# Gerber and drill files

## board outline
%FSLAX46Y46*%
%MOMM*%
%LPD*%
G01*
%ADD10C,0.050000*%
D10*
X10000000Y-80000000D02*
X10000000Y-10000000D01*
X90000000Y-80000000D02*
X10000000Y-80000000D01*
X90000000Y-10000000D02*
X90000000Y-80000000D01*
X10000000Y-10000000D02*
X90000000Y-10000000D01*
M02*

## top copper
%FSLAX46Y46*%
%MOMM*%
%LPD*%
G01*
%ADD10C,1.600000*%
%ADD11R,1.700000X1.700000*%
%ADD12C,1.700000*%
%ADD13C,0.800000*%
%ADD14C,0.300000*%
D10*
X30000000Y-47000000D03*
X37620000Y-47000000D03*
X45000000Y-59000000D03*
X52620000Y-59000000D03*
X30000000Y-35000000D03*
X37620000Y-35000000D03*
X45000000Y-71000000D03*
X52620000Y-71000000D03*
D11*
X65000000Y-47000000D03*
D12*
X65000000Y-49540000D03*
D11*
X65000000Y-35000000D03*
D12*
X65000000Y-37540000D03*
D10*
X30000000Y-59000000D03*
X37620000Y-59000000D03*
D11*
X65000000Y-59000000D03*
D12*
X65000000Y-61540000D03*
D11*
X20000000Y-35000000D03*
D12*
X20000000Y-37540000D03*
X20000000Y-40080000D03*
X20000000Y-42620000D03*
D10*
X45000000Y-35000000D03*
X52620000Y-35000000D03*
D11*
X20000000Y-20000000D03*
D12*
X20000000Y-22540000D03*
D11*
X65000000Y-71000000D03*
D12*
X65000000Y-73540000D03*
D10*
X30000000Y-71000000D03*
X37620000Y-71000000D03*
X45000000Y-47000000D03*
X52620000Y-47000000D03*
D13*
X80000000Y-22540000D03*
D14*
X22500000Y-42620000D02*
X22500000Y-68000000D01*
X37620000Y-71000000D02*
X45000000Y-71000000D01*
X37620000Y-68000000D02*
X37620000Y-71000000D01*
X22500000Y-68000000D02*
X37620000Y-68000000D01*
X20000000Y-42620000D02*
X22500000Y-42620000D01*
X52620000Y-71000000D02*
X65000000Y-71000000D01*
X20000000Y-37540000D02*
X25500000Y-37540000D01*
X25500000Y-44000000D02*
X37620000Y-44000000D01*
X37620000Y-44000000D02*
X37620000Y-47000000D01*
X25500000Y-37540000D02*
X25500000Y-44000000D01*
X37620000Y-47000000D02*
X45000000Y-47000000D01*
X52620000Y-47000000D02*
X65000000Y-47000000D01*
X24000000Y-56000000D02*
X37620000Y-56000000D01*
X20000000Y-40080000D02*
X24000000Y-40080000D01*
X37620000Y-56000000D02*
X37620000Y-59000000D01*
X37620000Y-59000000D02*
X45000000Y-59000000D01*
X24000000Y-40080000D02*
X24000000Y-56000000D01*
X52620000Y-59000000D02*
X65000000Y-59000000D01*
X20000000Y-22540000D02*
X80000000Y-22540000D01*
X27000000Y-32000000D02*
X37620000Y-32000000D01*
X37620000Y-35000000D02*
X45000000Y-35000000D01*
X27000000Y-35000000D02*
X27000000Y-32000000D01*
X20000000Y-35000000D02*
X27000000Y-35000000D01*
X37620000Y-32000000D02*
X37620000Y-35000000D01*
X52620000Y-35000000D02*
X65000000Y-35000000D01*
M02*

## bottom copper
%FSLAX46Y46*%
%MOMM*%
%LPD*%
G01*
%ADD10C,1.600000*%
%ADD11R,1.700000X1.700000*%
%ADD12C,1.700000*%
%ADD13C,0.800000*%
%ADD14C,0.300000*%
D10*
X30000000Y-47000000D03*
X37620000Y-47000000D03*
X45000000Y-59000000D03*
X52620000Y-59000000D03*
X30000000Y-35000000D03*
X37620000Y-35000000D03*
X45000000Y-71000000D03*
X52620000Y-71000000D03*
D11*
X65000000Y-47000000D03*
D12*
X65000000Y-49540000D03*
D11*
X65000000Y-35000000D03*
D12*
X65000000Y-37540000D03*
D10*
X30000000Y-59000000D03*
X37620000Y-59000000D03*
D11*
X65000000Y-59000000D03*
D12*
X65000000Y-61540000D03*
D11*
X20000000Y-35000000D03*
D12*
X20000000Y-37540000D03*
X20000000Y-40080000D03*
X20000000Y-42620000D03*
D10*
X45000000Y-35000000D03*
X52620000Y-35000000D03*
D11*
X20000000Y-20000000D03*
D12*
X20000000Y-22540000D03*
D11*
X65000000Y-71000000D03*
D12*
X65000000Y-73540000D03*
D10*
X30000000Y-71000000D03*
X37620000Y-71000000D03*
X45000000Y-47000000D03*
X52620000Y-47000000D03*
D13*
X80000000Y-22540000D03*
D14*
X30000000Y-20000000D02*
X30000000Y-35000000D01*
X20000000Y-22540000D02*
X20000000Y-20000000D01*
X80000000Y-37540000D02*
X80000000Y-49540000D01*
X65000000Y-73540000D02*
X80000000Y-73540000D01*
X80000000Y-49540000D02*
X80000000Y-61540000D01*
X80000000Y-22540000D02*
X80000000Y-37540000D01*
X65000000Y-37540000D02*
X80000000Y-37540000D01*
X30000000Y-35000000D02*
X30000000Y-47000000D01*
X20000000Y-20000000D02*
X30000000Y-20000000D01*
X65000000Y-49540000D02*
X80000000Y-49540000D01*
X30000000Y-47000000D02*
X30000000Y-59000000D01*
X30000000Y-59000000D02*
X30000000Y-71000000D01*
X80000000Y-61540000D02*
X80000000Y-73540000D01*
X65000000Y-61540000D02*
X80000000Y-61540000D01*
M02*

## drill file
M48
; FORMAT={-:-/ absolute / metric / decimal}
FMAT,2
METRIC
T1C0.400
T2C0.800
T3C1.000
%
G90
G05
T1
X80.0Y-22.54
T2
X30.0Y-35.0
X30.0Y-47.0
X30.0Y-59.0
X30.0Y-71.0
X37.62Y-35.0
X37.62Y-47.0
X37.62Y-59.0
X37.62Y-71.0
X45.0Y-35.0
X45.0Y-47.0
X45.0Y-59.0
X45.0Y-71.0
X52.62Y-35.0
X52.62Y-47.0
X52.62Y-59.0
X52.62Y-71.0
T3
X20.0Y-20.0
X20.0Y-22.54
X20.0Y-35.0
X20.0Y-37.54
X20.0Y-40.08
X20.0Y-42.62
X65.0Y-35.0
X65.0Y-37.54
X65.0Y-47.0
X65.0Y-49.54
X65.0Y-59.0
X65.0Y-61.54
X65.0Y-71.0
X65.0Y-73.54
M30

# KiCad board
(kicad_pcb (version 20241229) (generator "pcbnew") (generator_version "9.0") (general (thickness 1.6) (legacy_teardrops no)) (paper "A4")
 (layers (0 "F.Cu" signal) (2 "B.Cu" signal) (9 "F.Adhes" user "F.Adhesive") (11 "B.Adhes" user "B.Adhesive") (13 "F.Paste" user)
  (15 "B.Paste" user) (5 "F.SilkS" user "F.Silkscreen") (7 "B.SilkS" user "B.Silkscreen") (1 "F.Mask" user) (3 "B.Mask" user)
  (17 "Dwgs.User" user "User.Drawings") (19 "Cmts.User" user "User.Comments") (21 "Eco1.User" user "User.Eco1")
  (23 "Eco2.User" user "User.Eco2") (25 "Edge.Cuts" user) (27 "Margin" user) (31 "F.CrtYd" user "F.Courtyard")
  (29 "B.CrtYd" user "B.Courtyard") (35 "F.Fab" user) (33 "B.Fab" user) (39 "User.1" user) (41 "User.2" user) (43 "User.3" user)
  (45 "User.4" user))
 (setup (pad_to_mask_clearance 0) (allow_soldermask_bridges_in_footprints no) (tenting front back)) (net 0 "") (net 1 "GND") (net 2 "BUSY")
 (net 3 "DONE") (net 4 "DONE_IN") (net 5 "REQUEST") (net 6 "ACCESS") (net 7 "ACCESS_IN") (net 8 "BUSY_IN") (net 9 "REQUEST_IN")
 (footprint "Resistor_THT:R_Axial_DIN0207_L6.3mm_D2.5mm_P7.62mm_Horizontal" (layer "F.Cu") (at 30 47)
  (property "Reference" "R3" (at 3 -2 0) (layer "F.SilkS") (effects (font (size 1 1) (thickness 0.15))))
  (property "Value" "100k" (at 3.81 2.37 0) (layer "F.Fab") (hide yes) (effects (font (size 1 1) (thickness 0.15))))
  (pad "1" thru_hole circle (at 0 0) (size 1.6 1.6) (drill 0.8) (layers "*.Cu" "*.Mask") (remove_unused_layers no) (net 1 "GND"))
  (pad "2" thru_hole circle (at 7.62 0) (size 1.6 1.6) (drill 0.8) (layers "*.Cu" "*.Mask") (remove_unused_layers no) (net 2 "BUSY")))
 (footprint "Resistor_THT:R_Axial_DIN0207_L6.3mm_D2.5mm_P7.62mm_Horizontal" (layer "F.Cu") (at 45 59)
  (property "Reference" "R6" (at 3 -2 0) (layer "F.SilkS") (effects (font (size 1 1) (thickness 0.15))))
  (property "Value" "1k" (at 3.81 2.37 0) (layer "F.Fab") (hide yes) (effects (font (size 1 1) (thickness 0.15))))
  (pad "1" thru_hole circle (at 0 0) (size 1.6 1.6) (drill 0.8) (layers "*.Cu" "*.Mask") (remove_unused_layers no) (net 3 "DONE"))
  (pad "2" thru_hole circle (at 7.62 0) (size 1.6 1.6) (drill 0.8) (layers "*.Cu" "*.Mask") (remove_unused_layers no) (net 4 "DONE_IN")))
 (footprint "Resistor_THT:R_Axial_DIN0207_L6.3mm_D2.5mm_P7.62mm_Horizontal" (layer "F.Cu") (at 30 35)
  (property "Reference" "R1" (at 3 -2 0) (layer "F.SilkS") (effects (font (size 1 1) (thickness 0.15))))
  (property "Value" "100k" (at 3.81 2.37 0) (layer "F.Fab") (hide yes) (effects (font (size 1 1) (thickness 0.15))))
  (pad "1" thru_hole circle (at 0 0) (size 1.6 1.6) (drill 0.8) (layers "*.Cu" "*.Mask") (remove_unused_layers no) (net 1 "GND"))
  (pad "2" thru_hole circle (at 7.62 0) (size 1.6 1.6) (drill 0.8) (layers "*.Cu" "*.Mask") (remove_unused_layers no) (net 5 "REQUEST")))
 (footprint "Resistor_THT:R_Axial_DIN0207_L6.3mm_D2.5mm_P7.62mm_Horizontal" (layer "F.Cu") (at 45 71)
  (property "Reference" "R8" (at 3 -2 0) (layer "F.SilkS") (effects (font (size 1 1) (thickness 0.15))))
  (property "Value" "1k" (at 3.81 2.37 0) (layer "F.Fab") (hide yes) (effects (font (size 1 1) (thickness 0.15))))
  (pad "1" thru_hole circle (at 0 0) (size 1.6 1.6) (drill 0.8) (layers "*.Cu" "*.Mask") (remove_unused_layers no) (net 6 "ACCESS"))
  (pad "2" thru_hole circle (at 7.62 0) (size 1.6 1.6) (drill 0.8) (layers "*.Cu" "*.Mask") (remove_unused_layers no) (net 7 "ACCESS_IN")))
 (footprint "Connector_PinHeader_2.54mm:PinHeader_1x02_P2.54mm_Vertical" (layer "F.Cu") (at 65 47)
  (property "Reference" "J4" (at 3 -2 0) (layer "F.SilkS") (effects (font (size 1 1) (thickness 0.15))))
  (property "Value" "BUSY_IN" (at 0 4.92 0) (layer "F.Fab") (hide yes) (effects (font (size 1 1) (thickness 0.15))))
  (pad "1" thru_hole rect (at 0 0) (size 1.7 1.7) (drill 1) (layers "*.Cu" "*.Mask") (remove_unused_layers no) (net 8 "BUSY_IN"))
  (pad "2" thru_hole circle (at 0 2.54) (size 1.7 1.7) (drill 1) (layers "*.Cu" "*.Mask") (remove_unused_layers no) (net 1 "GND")))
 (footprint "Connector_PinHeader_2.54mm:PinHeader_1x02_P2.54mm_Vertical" (layer "F.Cu") (at 65 35)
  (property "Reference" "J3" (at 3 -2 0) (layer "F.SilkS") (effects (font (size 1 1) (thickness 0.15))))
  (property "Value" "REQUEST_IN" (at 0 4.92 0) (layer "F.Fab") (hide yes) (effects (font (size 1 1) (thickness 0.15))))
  (pad "1" thru_hole rect (at 0 0) (size 1.7 1.7) (drill 1) (layers "*.Cu" "*.Mask") (remove_unused_layers no) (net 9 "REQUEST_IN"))
  (pad "2" thru_hole circle (at 0 2.54) (size 1.7 1.7) (drill 1) (layers "*.Cu" "*.Mask") (remove_unused_layers no) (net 1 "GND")))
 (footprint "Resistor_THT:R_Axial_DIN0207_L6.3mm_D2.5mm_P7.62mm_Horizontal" (layer "F.Cu") (at 30 59)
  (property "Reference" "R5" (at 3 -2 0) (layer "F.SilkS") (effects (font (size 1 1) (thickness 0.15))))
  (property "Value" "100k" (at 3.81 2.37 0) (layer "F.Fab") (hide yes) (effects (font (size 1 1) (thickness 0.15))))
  (pad "1" thru_hole circle (at 0 0) (size 1.6 1.6) (drill 0.8) (layers "*.Cu" "*.Mask") (remove_unused_layers no) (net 1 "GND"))
  (pad "2" thru_hole circle (at 7.62 0) (size 1.6 1.6) (drill 0.8) (layers "*.Cu" "*.Mask") (remove_unused_layers no) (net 3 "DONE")))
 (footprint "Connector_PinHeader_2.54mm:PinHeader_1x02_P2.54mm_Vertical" (layer "F.Cu") (at 65 59)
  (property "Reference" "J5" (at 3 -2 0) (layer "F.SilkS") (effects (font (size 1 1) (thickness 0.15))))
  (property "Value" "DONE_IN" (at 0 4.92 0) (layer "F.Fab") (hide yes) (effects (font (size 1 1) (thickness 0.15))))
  (pad "1" thru_hole rect (at 0 0) (size 1.7 1.7) (drill 1) (layers "*.Cu" "*.Mask") (remove_unused_layers no) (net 4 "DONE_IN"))
  (pad "2" thru_hole circle (at 0 2.54) (size 1.7 1.7) (drill 1) (layers "*.Cu" "*.Mask") (remove_unused_layers no) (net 1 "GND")))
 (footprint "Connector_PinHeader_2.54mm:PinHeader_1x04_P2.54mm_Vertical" (layer "F.Cu") (at 20 35)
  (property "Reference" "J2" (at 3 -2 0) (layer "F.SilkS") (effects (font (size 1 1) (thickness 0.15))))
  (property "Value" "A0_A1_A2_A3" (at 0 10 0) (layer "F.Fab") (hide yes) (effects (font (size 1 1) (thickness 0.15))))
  (pad "1" thru_hole rect (at 0 0) (size 1.7 1.7) (drill 1) (layers "*.Cu" "*.Mask") (remove_unused_layers no) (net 5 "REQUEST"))
  (pad "2" thru_hole circle (at 0 2.54) (size 1.7 1.7) (drill 1) (layers "*.Cu" "*.Mask") (remove_unused_layers no) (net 2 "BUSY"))
  (pad "3" thru_hole circle (at 0 5.08) (size 1.7 1.7) (drill 1) (layers "*.Cu" "*.Mask") (remove_unused_layers no) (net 3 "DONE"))
  (pad "4" thru_hole circle (at 0 7.62) (size 1.7 1.7) (drill 1) (layers "*.Cu" "*.Mask") (remove_unused_layers no) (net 6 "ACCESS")))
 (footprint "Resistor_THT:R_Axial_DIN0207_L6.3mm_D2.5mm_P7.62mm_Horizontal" (layer "F.Cu") (at 45 35)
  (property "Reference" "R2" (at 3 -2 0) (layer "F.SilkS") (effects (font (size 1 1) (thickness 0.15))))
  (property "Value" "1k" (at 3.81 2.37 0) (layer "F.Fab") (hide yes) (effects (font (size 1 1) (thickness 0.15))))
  (pad "1" thru_hole circle (at 0 0) (size 1.6 1.6) (drill 0.8) (layers "*.Cu" "*.Mask") (remove_unused_layers no) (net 5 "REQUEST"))
  (pad "2" thru_hole circle (at 7.62 0) (size 1.6 1.6) (drill 0.8) (layers "*.Cu" "*.Mask") (remove_unused_layers no) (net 9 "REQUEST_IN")))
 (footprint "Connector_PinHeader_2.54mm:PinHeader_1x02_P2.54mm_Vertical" (layer "F.Cu") (at 20 20)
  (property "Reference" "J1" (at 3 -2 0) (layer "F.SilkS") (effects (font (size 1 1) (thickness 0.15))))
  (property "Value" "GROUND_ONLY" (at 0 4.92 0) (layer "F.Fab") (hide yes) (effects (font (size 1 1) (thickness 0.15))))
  (pad "1" thru_hole rect (at 0 0) (size 1.7 1.7) (drill 1) (layers "*.Cu" "*.Mask") (remove_unused_layers no) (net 1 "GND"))
  (pad "2" thru_hole circle (at 0 2.54) (size 1.7 1.7) (drill 1) (layers "*.Cu" "*.Mask") (remove_unused_layers no) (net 1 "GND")))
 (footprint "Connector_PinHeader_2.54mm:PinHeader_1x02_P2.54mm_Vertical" (layer "F.Cu") (at 65 71)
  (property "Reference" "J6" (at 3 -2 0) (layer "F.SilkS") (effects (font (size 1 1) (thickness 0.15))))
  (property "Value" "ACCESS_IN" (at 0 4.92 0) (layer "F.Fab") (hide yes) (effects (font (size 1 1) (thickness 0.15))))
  (pad "1" thru_hole rect (at 0 0) (size 1.7 1.7) (drill 1) (layers "*.Cu" "*.Mask") (remove_unused_layers no) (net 7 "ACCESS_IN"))
  (pad "2" thru_hole circle (at 0 2.54) (size 1.7 1.7) (drill 1) (layers "*.Cu" "*.Mask") (remove_unused_layers no) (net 1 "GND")))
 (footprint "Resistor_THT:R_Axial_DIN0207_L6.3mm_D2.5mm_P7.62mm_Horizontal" (layer "F.Cu") (at 30 71)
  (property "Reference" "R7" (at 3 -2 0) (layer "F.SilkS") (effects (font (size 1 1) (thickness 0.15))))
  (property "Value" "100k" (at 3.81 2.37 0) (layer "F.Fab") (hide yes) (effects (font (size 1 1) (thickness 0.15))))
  (pad "1" thru_hole circle (at 0 0) (size 1.6 1.6) (drill 0.8) (layers "*.Cu" "*.Mask") (remove_unused_layers no) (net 1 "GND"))
  (pad "2" thru_hole circle (at 7.62 0) (size 1.6 1.6) (drill 0.8) (layers "*.Cu" "*.Mask") (remove_unused_layers no) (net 6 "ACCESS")))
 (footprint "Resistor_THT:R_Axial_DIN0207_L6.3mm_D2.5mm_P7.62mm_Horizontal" (layer "F.Cu") (at 45 47)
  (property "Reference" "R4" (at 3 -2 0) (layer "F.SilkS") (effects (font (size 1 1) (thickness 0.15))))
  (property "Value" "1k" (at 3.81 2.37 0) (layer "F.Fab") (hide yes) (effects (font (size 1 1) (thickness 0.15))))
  (pad "1" thru_hole circle (at 0 0) (size 1.6 1.6) (drill 0.8) (layers "*.Cu" "*.Mask") (remove_unused_layers no) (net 2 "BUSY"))
  (pad "2" thru_hole circle (at 7.62 0) (size 1.6 1.6) (drill 0.8) (layers "*.Cu" "*.Mask") (remove_unused_layers no) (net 8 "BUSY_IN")))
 (gr_line (start 10 80) (end 10 10) (stroke (width 0.05) (type default)) (layer "Edge.Cuts"))
 (gr_line (start 90 80) (end 10 80) (stroke (width 0.05) (type default)) (layer "Edge.Cuts"))
 (gr_line (start 90 10) (end 90 80) (stroke (width 0.05) (type default)) (layer "Edge.Cuts"))
 (gr_line (start 10 10) (end 90 10) (stroke (width 0.05) (type default)) (layer "Edge.Cuts"))
 (segment (start 22.5 42.62) (end 22.5 68) (width 0.3) (layer "F.Cu") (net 6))
 (segment (start 37.62 71) (end 45 71) (width 0.3) (layer "F.Cu") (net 6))
 (segment (start 37.62 68) (end 37.62 71) (width 0.3) (layer "F.Cu") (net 6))
 (segment (start 22.5 68) (end 37.62 68) (width 0.3) (layer "F.Cu") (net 6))
 (segment (start 20 42.62) (end 22.5 42.62) (width 0.3) (layer "F.Cu") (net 6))
 (segment (start 52.62 71) (end 65 71) (width 0.3) (layer "F.Cu") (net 7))
 (segment (start 20 37.54) (end 25.5 37.54) (width 0.3) (layer "F.Cu") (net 2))
 (segment (start 25.5 44) (end 37.62 44) (width 0.3) (layer "F.Cu") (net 2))
 (segment (start 37.62 44) (end 37.62 47) (width 0.3) (layer "F.Cu") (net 2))
 (segment (start 25.5 37.54) (end 25.5 44) (width 0.3) (layer "F.Cu") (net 2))
 (segment (start 37.62 47) (end 45 47) (width 0.3) (layer "F.Cu") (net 2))
 (segment (start 52.62 47) (end 65 47) (width 0.3) (layer "F.Cu") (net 8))
 (segment (start 24 56) (end 37.62 56) (width 0.3) (layer "F.Cu") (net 3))
 (segment (start 20 40.08) (end 24 40.08) (width 0.3) (layer "F.Cu") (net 3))
 (segment (start 37.62 56) (end 37.62 59) (width 0.3) (layer "F.Cu") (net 3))
 (segment (start 37.62 59) (end 45 59) (width 0.3) (layer "F.Cu") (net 3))
 (segment (start 24 40.08) (end 24 56) (width 0.3) (layer "F.Cu") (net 3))
 (segment (start 52.62 59) (end 65 59) (width 0.3) (layer "F.Cu") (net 4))
 (segment (start 20 22.54) (end 80 22.54) (width 0.3) (layer "F.Cu") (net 1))
 (via (at 80 22.54) (size 0.8) (drill 0.4) (layers "F.Cu" "B.Cu") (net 1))
 (segment (start 30 20) (end 30 35) (width 0.3) (layer "B.Cu") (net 1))
 (segment (start 20 22.54) (end 20 20) (width 0.3) (layer "B.Cu") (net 1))
 (segment (start 80 37.54) (end 80 49.54) (width 0.3) (layer "B.Cu") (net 1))
 (segment (start 65 73.54) (end 80 73.54) (width 0.3) (layer "B.Cu") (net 1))
 (segment (start 80 49.54) (end 80 61.54) (width 0.3) (layer "B.Cu") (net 1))
 (segment (start 80 22.54) (end 80 37.54) (width 0.3) (layer "B.Cu") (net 1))
 (segment (start 65 37.54) (end 80 37.54) (width 0.3) (layer "B.Cu") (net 1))
 (segment (start 30 35) (end 30 47) (width 0.3) (layer "B.Cu") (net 1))
 (segment (start 20 20) (end 30 20) (width 0.3) (layer "B.Cu") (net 1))
 (segment (start 65 49.54) (end 80 49.54) (width 0.3) (layer "B.Cu") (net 1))
 (segment (start 30 47) (end 30 59) (width 0.3) (layer "B.Cu") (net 1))
 (segment (start 30 59) (end 30 71) (width 0.3) (layer "B.Cu") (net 1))
 (segment (start 80 61.54) (end 80 73.54) (width 0.3) (layer "B.Cu") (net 1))
 (segment (start 65 61.54) (end 80 61.54) (width 0.3) (layer "B.Cu") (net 1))
 (segment (start 27 32) (end 37.62 32) (width 0.3) (layer "F.Cu") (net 5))
 (segment (start 37.62 35) (end 45 35) (width 0.3) (layer "F.Cu") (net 5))
 (segment (start 27 35) (end 27 32) (width 0.3) (layer "F.Cu") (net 5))
 (segment (start 20 35) (end 27 35) (width 0.3) (layer "F.Cu") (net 5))
 (segment (start 37.62 32) (end 37.62 35) (width 0.3) (layer "F.Cu") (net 5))
 (segment (start 52.62 35) (end 65 35) (width 0.3) (layer "F.Cu") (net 9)))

